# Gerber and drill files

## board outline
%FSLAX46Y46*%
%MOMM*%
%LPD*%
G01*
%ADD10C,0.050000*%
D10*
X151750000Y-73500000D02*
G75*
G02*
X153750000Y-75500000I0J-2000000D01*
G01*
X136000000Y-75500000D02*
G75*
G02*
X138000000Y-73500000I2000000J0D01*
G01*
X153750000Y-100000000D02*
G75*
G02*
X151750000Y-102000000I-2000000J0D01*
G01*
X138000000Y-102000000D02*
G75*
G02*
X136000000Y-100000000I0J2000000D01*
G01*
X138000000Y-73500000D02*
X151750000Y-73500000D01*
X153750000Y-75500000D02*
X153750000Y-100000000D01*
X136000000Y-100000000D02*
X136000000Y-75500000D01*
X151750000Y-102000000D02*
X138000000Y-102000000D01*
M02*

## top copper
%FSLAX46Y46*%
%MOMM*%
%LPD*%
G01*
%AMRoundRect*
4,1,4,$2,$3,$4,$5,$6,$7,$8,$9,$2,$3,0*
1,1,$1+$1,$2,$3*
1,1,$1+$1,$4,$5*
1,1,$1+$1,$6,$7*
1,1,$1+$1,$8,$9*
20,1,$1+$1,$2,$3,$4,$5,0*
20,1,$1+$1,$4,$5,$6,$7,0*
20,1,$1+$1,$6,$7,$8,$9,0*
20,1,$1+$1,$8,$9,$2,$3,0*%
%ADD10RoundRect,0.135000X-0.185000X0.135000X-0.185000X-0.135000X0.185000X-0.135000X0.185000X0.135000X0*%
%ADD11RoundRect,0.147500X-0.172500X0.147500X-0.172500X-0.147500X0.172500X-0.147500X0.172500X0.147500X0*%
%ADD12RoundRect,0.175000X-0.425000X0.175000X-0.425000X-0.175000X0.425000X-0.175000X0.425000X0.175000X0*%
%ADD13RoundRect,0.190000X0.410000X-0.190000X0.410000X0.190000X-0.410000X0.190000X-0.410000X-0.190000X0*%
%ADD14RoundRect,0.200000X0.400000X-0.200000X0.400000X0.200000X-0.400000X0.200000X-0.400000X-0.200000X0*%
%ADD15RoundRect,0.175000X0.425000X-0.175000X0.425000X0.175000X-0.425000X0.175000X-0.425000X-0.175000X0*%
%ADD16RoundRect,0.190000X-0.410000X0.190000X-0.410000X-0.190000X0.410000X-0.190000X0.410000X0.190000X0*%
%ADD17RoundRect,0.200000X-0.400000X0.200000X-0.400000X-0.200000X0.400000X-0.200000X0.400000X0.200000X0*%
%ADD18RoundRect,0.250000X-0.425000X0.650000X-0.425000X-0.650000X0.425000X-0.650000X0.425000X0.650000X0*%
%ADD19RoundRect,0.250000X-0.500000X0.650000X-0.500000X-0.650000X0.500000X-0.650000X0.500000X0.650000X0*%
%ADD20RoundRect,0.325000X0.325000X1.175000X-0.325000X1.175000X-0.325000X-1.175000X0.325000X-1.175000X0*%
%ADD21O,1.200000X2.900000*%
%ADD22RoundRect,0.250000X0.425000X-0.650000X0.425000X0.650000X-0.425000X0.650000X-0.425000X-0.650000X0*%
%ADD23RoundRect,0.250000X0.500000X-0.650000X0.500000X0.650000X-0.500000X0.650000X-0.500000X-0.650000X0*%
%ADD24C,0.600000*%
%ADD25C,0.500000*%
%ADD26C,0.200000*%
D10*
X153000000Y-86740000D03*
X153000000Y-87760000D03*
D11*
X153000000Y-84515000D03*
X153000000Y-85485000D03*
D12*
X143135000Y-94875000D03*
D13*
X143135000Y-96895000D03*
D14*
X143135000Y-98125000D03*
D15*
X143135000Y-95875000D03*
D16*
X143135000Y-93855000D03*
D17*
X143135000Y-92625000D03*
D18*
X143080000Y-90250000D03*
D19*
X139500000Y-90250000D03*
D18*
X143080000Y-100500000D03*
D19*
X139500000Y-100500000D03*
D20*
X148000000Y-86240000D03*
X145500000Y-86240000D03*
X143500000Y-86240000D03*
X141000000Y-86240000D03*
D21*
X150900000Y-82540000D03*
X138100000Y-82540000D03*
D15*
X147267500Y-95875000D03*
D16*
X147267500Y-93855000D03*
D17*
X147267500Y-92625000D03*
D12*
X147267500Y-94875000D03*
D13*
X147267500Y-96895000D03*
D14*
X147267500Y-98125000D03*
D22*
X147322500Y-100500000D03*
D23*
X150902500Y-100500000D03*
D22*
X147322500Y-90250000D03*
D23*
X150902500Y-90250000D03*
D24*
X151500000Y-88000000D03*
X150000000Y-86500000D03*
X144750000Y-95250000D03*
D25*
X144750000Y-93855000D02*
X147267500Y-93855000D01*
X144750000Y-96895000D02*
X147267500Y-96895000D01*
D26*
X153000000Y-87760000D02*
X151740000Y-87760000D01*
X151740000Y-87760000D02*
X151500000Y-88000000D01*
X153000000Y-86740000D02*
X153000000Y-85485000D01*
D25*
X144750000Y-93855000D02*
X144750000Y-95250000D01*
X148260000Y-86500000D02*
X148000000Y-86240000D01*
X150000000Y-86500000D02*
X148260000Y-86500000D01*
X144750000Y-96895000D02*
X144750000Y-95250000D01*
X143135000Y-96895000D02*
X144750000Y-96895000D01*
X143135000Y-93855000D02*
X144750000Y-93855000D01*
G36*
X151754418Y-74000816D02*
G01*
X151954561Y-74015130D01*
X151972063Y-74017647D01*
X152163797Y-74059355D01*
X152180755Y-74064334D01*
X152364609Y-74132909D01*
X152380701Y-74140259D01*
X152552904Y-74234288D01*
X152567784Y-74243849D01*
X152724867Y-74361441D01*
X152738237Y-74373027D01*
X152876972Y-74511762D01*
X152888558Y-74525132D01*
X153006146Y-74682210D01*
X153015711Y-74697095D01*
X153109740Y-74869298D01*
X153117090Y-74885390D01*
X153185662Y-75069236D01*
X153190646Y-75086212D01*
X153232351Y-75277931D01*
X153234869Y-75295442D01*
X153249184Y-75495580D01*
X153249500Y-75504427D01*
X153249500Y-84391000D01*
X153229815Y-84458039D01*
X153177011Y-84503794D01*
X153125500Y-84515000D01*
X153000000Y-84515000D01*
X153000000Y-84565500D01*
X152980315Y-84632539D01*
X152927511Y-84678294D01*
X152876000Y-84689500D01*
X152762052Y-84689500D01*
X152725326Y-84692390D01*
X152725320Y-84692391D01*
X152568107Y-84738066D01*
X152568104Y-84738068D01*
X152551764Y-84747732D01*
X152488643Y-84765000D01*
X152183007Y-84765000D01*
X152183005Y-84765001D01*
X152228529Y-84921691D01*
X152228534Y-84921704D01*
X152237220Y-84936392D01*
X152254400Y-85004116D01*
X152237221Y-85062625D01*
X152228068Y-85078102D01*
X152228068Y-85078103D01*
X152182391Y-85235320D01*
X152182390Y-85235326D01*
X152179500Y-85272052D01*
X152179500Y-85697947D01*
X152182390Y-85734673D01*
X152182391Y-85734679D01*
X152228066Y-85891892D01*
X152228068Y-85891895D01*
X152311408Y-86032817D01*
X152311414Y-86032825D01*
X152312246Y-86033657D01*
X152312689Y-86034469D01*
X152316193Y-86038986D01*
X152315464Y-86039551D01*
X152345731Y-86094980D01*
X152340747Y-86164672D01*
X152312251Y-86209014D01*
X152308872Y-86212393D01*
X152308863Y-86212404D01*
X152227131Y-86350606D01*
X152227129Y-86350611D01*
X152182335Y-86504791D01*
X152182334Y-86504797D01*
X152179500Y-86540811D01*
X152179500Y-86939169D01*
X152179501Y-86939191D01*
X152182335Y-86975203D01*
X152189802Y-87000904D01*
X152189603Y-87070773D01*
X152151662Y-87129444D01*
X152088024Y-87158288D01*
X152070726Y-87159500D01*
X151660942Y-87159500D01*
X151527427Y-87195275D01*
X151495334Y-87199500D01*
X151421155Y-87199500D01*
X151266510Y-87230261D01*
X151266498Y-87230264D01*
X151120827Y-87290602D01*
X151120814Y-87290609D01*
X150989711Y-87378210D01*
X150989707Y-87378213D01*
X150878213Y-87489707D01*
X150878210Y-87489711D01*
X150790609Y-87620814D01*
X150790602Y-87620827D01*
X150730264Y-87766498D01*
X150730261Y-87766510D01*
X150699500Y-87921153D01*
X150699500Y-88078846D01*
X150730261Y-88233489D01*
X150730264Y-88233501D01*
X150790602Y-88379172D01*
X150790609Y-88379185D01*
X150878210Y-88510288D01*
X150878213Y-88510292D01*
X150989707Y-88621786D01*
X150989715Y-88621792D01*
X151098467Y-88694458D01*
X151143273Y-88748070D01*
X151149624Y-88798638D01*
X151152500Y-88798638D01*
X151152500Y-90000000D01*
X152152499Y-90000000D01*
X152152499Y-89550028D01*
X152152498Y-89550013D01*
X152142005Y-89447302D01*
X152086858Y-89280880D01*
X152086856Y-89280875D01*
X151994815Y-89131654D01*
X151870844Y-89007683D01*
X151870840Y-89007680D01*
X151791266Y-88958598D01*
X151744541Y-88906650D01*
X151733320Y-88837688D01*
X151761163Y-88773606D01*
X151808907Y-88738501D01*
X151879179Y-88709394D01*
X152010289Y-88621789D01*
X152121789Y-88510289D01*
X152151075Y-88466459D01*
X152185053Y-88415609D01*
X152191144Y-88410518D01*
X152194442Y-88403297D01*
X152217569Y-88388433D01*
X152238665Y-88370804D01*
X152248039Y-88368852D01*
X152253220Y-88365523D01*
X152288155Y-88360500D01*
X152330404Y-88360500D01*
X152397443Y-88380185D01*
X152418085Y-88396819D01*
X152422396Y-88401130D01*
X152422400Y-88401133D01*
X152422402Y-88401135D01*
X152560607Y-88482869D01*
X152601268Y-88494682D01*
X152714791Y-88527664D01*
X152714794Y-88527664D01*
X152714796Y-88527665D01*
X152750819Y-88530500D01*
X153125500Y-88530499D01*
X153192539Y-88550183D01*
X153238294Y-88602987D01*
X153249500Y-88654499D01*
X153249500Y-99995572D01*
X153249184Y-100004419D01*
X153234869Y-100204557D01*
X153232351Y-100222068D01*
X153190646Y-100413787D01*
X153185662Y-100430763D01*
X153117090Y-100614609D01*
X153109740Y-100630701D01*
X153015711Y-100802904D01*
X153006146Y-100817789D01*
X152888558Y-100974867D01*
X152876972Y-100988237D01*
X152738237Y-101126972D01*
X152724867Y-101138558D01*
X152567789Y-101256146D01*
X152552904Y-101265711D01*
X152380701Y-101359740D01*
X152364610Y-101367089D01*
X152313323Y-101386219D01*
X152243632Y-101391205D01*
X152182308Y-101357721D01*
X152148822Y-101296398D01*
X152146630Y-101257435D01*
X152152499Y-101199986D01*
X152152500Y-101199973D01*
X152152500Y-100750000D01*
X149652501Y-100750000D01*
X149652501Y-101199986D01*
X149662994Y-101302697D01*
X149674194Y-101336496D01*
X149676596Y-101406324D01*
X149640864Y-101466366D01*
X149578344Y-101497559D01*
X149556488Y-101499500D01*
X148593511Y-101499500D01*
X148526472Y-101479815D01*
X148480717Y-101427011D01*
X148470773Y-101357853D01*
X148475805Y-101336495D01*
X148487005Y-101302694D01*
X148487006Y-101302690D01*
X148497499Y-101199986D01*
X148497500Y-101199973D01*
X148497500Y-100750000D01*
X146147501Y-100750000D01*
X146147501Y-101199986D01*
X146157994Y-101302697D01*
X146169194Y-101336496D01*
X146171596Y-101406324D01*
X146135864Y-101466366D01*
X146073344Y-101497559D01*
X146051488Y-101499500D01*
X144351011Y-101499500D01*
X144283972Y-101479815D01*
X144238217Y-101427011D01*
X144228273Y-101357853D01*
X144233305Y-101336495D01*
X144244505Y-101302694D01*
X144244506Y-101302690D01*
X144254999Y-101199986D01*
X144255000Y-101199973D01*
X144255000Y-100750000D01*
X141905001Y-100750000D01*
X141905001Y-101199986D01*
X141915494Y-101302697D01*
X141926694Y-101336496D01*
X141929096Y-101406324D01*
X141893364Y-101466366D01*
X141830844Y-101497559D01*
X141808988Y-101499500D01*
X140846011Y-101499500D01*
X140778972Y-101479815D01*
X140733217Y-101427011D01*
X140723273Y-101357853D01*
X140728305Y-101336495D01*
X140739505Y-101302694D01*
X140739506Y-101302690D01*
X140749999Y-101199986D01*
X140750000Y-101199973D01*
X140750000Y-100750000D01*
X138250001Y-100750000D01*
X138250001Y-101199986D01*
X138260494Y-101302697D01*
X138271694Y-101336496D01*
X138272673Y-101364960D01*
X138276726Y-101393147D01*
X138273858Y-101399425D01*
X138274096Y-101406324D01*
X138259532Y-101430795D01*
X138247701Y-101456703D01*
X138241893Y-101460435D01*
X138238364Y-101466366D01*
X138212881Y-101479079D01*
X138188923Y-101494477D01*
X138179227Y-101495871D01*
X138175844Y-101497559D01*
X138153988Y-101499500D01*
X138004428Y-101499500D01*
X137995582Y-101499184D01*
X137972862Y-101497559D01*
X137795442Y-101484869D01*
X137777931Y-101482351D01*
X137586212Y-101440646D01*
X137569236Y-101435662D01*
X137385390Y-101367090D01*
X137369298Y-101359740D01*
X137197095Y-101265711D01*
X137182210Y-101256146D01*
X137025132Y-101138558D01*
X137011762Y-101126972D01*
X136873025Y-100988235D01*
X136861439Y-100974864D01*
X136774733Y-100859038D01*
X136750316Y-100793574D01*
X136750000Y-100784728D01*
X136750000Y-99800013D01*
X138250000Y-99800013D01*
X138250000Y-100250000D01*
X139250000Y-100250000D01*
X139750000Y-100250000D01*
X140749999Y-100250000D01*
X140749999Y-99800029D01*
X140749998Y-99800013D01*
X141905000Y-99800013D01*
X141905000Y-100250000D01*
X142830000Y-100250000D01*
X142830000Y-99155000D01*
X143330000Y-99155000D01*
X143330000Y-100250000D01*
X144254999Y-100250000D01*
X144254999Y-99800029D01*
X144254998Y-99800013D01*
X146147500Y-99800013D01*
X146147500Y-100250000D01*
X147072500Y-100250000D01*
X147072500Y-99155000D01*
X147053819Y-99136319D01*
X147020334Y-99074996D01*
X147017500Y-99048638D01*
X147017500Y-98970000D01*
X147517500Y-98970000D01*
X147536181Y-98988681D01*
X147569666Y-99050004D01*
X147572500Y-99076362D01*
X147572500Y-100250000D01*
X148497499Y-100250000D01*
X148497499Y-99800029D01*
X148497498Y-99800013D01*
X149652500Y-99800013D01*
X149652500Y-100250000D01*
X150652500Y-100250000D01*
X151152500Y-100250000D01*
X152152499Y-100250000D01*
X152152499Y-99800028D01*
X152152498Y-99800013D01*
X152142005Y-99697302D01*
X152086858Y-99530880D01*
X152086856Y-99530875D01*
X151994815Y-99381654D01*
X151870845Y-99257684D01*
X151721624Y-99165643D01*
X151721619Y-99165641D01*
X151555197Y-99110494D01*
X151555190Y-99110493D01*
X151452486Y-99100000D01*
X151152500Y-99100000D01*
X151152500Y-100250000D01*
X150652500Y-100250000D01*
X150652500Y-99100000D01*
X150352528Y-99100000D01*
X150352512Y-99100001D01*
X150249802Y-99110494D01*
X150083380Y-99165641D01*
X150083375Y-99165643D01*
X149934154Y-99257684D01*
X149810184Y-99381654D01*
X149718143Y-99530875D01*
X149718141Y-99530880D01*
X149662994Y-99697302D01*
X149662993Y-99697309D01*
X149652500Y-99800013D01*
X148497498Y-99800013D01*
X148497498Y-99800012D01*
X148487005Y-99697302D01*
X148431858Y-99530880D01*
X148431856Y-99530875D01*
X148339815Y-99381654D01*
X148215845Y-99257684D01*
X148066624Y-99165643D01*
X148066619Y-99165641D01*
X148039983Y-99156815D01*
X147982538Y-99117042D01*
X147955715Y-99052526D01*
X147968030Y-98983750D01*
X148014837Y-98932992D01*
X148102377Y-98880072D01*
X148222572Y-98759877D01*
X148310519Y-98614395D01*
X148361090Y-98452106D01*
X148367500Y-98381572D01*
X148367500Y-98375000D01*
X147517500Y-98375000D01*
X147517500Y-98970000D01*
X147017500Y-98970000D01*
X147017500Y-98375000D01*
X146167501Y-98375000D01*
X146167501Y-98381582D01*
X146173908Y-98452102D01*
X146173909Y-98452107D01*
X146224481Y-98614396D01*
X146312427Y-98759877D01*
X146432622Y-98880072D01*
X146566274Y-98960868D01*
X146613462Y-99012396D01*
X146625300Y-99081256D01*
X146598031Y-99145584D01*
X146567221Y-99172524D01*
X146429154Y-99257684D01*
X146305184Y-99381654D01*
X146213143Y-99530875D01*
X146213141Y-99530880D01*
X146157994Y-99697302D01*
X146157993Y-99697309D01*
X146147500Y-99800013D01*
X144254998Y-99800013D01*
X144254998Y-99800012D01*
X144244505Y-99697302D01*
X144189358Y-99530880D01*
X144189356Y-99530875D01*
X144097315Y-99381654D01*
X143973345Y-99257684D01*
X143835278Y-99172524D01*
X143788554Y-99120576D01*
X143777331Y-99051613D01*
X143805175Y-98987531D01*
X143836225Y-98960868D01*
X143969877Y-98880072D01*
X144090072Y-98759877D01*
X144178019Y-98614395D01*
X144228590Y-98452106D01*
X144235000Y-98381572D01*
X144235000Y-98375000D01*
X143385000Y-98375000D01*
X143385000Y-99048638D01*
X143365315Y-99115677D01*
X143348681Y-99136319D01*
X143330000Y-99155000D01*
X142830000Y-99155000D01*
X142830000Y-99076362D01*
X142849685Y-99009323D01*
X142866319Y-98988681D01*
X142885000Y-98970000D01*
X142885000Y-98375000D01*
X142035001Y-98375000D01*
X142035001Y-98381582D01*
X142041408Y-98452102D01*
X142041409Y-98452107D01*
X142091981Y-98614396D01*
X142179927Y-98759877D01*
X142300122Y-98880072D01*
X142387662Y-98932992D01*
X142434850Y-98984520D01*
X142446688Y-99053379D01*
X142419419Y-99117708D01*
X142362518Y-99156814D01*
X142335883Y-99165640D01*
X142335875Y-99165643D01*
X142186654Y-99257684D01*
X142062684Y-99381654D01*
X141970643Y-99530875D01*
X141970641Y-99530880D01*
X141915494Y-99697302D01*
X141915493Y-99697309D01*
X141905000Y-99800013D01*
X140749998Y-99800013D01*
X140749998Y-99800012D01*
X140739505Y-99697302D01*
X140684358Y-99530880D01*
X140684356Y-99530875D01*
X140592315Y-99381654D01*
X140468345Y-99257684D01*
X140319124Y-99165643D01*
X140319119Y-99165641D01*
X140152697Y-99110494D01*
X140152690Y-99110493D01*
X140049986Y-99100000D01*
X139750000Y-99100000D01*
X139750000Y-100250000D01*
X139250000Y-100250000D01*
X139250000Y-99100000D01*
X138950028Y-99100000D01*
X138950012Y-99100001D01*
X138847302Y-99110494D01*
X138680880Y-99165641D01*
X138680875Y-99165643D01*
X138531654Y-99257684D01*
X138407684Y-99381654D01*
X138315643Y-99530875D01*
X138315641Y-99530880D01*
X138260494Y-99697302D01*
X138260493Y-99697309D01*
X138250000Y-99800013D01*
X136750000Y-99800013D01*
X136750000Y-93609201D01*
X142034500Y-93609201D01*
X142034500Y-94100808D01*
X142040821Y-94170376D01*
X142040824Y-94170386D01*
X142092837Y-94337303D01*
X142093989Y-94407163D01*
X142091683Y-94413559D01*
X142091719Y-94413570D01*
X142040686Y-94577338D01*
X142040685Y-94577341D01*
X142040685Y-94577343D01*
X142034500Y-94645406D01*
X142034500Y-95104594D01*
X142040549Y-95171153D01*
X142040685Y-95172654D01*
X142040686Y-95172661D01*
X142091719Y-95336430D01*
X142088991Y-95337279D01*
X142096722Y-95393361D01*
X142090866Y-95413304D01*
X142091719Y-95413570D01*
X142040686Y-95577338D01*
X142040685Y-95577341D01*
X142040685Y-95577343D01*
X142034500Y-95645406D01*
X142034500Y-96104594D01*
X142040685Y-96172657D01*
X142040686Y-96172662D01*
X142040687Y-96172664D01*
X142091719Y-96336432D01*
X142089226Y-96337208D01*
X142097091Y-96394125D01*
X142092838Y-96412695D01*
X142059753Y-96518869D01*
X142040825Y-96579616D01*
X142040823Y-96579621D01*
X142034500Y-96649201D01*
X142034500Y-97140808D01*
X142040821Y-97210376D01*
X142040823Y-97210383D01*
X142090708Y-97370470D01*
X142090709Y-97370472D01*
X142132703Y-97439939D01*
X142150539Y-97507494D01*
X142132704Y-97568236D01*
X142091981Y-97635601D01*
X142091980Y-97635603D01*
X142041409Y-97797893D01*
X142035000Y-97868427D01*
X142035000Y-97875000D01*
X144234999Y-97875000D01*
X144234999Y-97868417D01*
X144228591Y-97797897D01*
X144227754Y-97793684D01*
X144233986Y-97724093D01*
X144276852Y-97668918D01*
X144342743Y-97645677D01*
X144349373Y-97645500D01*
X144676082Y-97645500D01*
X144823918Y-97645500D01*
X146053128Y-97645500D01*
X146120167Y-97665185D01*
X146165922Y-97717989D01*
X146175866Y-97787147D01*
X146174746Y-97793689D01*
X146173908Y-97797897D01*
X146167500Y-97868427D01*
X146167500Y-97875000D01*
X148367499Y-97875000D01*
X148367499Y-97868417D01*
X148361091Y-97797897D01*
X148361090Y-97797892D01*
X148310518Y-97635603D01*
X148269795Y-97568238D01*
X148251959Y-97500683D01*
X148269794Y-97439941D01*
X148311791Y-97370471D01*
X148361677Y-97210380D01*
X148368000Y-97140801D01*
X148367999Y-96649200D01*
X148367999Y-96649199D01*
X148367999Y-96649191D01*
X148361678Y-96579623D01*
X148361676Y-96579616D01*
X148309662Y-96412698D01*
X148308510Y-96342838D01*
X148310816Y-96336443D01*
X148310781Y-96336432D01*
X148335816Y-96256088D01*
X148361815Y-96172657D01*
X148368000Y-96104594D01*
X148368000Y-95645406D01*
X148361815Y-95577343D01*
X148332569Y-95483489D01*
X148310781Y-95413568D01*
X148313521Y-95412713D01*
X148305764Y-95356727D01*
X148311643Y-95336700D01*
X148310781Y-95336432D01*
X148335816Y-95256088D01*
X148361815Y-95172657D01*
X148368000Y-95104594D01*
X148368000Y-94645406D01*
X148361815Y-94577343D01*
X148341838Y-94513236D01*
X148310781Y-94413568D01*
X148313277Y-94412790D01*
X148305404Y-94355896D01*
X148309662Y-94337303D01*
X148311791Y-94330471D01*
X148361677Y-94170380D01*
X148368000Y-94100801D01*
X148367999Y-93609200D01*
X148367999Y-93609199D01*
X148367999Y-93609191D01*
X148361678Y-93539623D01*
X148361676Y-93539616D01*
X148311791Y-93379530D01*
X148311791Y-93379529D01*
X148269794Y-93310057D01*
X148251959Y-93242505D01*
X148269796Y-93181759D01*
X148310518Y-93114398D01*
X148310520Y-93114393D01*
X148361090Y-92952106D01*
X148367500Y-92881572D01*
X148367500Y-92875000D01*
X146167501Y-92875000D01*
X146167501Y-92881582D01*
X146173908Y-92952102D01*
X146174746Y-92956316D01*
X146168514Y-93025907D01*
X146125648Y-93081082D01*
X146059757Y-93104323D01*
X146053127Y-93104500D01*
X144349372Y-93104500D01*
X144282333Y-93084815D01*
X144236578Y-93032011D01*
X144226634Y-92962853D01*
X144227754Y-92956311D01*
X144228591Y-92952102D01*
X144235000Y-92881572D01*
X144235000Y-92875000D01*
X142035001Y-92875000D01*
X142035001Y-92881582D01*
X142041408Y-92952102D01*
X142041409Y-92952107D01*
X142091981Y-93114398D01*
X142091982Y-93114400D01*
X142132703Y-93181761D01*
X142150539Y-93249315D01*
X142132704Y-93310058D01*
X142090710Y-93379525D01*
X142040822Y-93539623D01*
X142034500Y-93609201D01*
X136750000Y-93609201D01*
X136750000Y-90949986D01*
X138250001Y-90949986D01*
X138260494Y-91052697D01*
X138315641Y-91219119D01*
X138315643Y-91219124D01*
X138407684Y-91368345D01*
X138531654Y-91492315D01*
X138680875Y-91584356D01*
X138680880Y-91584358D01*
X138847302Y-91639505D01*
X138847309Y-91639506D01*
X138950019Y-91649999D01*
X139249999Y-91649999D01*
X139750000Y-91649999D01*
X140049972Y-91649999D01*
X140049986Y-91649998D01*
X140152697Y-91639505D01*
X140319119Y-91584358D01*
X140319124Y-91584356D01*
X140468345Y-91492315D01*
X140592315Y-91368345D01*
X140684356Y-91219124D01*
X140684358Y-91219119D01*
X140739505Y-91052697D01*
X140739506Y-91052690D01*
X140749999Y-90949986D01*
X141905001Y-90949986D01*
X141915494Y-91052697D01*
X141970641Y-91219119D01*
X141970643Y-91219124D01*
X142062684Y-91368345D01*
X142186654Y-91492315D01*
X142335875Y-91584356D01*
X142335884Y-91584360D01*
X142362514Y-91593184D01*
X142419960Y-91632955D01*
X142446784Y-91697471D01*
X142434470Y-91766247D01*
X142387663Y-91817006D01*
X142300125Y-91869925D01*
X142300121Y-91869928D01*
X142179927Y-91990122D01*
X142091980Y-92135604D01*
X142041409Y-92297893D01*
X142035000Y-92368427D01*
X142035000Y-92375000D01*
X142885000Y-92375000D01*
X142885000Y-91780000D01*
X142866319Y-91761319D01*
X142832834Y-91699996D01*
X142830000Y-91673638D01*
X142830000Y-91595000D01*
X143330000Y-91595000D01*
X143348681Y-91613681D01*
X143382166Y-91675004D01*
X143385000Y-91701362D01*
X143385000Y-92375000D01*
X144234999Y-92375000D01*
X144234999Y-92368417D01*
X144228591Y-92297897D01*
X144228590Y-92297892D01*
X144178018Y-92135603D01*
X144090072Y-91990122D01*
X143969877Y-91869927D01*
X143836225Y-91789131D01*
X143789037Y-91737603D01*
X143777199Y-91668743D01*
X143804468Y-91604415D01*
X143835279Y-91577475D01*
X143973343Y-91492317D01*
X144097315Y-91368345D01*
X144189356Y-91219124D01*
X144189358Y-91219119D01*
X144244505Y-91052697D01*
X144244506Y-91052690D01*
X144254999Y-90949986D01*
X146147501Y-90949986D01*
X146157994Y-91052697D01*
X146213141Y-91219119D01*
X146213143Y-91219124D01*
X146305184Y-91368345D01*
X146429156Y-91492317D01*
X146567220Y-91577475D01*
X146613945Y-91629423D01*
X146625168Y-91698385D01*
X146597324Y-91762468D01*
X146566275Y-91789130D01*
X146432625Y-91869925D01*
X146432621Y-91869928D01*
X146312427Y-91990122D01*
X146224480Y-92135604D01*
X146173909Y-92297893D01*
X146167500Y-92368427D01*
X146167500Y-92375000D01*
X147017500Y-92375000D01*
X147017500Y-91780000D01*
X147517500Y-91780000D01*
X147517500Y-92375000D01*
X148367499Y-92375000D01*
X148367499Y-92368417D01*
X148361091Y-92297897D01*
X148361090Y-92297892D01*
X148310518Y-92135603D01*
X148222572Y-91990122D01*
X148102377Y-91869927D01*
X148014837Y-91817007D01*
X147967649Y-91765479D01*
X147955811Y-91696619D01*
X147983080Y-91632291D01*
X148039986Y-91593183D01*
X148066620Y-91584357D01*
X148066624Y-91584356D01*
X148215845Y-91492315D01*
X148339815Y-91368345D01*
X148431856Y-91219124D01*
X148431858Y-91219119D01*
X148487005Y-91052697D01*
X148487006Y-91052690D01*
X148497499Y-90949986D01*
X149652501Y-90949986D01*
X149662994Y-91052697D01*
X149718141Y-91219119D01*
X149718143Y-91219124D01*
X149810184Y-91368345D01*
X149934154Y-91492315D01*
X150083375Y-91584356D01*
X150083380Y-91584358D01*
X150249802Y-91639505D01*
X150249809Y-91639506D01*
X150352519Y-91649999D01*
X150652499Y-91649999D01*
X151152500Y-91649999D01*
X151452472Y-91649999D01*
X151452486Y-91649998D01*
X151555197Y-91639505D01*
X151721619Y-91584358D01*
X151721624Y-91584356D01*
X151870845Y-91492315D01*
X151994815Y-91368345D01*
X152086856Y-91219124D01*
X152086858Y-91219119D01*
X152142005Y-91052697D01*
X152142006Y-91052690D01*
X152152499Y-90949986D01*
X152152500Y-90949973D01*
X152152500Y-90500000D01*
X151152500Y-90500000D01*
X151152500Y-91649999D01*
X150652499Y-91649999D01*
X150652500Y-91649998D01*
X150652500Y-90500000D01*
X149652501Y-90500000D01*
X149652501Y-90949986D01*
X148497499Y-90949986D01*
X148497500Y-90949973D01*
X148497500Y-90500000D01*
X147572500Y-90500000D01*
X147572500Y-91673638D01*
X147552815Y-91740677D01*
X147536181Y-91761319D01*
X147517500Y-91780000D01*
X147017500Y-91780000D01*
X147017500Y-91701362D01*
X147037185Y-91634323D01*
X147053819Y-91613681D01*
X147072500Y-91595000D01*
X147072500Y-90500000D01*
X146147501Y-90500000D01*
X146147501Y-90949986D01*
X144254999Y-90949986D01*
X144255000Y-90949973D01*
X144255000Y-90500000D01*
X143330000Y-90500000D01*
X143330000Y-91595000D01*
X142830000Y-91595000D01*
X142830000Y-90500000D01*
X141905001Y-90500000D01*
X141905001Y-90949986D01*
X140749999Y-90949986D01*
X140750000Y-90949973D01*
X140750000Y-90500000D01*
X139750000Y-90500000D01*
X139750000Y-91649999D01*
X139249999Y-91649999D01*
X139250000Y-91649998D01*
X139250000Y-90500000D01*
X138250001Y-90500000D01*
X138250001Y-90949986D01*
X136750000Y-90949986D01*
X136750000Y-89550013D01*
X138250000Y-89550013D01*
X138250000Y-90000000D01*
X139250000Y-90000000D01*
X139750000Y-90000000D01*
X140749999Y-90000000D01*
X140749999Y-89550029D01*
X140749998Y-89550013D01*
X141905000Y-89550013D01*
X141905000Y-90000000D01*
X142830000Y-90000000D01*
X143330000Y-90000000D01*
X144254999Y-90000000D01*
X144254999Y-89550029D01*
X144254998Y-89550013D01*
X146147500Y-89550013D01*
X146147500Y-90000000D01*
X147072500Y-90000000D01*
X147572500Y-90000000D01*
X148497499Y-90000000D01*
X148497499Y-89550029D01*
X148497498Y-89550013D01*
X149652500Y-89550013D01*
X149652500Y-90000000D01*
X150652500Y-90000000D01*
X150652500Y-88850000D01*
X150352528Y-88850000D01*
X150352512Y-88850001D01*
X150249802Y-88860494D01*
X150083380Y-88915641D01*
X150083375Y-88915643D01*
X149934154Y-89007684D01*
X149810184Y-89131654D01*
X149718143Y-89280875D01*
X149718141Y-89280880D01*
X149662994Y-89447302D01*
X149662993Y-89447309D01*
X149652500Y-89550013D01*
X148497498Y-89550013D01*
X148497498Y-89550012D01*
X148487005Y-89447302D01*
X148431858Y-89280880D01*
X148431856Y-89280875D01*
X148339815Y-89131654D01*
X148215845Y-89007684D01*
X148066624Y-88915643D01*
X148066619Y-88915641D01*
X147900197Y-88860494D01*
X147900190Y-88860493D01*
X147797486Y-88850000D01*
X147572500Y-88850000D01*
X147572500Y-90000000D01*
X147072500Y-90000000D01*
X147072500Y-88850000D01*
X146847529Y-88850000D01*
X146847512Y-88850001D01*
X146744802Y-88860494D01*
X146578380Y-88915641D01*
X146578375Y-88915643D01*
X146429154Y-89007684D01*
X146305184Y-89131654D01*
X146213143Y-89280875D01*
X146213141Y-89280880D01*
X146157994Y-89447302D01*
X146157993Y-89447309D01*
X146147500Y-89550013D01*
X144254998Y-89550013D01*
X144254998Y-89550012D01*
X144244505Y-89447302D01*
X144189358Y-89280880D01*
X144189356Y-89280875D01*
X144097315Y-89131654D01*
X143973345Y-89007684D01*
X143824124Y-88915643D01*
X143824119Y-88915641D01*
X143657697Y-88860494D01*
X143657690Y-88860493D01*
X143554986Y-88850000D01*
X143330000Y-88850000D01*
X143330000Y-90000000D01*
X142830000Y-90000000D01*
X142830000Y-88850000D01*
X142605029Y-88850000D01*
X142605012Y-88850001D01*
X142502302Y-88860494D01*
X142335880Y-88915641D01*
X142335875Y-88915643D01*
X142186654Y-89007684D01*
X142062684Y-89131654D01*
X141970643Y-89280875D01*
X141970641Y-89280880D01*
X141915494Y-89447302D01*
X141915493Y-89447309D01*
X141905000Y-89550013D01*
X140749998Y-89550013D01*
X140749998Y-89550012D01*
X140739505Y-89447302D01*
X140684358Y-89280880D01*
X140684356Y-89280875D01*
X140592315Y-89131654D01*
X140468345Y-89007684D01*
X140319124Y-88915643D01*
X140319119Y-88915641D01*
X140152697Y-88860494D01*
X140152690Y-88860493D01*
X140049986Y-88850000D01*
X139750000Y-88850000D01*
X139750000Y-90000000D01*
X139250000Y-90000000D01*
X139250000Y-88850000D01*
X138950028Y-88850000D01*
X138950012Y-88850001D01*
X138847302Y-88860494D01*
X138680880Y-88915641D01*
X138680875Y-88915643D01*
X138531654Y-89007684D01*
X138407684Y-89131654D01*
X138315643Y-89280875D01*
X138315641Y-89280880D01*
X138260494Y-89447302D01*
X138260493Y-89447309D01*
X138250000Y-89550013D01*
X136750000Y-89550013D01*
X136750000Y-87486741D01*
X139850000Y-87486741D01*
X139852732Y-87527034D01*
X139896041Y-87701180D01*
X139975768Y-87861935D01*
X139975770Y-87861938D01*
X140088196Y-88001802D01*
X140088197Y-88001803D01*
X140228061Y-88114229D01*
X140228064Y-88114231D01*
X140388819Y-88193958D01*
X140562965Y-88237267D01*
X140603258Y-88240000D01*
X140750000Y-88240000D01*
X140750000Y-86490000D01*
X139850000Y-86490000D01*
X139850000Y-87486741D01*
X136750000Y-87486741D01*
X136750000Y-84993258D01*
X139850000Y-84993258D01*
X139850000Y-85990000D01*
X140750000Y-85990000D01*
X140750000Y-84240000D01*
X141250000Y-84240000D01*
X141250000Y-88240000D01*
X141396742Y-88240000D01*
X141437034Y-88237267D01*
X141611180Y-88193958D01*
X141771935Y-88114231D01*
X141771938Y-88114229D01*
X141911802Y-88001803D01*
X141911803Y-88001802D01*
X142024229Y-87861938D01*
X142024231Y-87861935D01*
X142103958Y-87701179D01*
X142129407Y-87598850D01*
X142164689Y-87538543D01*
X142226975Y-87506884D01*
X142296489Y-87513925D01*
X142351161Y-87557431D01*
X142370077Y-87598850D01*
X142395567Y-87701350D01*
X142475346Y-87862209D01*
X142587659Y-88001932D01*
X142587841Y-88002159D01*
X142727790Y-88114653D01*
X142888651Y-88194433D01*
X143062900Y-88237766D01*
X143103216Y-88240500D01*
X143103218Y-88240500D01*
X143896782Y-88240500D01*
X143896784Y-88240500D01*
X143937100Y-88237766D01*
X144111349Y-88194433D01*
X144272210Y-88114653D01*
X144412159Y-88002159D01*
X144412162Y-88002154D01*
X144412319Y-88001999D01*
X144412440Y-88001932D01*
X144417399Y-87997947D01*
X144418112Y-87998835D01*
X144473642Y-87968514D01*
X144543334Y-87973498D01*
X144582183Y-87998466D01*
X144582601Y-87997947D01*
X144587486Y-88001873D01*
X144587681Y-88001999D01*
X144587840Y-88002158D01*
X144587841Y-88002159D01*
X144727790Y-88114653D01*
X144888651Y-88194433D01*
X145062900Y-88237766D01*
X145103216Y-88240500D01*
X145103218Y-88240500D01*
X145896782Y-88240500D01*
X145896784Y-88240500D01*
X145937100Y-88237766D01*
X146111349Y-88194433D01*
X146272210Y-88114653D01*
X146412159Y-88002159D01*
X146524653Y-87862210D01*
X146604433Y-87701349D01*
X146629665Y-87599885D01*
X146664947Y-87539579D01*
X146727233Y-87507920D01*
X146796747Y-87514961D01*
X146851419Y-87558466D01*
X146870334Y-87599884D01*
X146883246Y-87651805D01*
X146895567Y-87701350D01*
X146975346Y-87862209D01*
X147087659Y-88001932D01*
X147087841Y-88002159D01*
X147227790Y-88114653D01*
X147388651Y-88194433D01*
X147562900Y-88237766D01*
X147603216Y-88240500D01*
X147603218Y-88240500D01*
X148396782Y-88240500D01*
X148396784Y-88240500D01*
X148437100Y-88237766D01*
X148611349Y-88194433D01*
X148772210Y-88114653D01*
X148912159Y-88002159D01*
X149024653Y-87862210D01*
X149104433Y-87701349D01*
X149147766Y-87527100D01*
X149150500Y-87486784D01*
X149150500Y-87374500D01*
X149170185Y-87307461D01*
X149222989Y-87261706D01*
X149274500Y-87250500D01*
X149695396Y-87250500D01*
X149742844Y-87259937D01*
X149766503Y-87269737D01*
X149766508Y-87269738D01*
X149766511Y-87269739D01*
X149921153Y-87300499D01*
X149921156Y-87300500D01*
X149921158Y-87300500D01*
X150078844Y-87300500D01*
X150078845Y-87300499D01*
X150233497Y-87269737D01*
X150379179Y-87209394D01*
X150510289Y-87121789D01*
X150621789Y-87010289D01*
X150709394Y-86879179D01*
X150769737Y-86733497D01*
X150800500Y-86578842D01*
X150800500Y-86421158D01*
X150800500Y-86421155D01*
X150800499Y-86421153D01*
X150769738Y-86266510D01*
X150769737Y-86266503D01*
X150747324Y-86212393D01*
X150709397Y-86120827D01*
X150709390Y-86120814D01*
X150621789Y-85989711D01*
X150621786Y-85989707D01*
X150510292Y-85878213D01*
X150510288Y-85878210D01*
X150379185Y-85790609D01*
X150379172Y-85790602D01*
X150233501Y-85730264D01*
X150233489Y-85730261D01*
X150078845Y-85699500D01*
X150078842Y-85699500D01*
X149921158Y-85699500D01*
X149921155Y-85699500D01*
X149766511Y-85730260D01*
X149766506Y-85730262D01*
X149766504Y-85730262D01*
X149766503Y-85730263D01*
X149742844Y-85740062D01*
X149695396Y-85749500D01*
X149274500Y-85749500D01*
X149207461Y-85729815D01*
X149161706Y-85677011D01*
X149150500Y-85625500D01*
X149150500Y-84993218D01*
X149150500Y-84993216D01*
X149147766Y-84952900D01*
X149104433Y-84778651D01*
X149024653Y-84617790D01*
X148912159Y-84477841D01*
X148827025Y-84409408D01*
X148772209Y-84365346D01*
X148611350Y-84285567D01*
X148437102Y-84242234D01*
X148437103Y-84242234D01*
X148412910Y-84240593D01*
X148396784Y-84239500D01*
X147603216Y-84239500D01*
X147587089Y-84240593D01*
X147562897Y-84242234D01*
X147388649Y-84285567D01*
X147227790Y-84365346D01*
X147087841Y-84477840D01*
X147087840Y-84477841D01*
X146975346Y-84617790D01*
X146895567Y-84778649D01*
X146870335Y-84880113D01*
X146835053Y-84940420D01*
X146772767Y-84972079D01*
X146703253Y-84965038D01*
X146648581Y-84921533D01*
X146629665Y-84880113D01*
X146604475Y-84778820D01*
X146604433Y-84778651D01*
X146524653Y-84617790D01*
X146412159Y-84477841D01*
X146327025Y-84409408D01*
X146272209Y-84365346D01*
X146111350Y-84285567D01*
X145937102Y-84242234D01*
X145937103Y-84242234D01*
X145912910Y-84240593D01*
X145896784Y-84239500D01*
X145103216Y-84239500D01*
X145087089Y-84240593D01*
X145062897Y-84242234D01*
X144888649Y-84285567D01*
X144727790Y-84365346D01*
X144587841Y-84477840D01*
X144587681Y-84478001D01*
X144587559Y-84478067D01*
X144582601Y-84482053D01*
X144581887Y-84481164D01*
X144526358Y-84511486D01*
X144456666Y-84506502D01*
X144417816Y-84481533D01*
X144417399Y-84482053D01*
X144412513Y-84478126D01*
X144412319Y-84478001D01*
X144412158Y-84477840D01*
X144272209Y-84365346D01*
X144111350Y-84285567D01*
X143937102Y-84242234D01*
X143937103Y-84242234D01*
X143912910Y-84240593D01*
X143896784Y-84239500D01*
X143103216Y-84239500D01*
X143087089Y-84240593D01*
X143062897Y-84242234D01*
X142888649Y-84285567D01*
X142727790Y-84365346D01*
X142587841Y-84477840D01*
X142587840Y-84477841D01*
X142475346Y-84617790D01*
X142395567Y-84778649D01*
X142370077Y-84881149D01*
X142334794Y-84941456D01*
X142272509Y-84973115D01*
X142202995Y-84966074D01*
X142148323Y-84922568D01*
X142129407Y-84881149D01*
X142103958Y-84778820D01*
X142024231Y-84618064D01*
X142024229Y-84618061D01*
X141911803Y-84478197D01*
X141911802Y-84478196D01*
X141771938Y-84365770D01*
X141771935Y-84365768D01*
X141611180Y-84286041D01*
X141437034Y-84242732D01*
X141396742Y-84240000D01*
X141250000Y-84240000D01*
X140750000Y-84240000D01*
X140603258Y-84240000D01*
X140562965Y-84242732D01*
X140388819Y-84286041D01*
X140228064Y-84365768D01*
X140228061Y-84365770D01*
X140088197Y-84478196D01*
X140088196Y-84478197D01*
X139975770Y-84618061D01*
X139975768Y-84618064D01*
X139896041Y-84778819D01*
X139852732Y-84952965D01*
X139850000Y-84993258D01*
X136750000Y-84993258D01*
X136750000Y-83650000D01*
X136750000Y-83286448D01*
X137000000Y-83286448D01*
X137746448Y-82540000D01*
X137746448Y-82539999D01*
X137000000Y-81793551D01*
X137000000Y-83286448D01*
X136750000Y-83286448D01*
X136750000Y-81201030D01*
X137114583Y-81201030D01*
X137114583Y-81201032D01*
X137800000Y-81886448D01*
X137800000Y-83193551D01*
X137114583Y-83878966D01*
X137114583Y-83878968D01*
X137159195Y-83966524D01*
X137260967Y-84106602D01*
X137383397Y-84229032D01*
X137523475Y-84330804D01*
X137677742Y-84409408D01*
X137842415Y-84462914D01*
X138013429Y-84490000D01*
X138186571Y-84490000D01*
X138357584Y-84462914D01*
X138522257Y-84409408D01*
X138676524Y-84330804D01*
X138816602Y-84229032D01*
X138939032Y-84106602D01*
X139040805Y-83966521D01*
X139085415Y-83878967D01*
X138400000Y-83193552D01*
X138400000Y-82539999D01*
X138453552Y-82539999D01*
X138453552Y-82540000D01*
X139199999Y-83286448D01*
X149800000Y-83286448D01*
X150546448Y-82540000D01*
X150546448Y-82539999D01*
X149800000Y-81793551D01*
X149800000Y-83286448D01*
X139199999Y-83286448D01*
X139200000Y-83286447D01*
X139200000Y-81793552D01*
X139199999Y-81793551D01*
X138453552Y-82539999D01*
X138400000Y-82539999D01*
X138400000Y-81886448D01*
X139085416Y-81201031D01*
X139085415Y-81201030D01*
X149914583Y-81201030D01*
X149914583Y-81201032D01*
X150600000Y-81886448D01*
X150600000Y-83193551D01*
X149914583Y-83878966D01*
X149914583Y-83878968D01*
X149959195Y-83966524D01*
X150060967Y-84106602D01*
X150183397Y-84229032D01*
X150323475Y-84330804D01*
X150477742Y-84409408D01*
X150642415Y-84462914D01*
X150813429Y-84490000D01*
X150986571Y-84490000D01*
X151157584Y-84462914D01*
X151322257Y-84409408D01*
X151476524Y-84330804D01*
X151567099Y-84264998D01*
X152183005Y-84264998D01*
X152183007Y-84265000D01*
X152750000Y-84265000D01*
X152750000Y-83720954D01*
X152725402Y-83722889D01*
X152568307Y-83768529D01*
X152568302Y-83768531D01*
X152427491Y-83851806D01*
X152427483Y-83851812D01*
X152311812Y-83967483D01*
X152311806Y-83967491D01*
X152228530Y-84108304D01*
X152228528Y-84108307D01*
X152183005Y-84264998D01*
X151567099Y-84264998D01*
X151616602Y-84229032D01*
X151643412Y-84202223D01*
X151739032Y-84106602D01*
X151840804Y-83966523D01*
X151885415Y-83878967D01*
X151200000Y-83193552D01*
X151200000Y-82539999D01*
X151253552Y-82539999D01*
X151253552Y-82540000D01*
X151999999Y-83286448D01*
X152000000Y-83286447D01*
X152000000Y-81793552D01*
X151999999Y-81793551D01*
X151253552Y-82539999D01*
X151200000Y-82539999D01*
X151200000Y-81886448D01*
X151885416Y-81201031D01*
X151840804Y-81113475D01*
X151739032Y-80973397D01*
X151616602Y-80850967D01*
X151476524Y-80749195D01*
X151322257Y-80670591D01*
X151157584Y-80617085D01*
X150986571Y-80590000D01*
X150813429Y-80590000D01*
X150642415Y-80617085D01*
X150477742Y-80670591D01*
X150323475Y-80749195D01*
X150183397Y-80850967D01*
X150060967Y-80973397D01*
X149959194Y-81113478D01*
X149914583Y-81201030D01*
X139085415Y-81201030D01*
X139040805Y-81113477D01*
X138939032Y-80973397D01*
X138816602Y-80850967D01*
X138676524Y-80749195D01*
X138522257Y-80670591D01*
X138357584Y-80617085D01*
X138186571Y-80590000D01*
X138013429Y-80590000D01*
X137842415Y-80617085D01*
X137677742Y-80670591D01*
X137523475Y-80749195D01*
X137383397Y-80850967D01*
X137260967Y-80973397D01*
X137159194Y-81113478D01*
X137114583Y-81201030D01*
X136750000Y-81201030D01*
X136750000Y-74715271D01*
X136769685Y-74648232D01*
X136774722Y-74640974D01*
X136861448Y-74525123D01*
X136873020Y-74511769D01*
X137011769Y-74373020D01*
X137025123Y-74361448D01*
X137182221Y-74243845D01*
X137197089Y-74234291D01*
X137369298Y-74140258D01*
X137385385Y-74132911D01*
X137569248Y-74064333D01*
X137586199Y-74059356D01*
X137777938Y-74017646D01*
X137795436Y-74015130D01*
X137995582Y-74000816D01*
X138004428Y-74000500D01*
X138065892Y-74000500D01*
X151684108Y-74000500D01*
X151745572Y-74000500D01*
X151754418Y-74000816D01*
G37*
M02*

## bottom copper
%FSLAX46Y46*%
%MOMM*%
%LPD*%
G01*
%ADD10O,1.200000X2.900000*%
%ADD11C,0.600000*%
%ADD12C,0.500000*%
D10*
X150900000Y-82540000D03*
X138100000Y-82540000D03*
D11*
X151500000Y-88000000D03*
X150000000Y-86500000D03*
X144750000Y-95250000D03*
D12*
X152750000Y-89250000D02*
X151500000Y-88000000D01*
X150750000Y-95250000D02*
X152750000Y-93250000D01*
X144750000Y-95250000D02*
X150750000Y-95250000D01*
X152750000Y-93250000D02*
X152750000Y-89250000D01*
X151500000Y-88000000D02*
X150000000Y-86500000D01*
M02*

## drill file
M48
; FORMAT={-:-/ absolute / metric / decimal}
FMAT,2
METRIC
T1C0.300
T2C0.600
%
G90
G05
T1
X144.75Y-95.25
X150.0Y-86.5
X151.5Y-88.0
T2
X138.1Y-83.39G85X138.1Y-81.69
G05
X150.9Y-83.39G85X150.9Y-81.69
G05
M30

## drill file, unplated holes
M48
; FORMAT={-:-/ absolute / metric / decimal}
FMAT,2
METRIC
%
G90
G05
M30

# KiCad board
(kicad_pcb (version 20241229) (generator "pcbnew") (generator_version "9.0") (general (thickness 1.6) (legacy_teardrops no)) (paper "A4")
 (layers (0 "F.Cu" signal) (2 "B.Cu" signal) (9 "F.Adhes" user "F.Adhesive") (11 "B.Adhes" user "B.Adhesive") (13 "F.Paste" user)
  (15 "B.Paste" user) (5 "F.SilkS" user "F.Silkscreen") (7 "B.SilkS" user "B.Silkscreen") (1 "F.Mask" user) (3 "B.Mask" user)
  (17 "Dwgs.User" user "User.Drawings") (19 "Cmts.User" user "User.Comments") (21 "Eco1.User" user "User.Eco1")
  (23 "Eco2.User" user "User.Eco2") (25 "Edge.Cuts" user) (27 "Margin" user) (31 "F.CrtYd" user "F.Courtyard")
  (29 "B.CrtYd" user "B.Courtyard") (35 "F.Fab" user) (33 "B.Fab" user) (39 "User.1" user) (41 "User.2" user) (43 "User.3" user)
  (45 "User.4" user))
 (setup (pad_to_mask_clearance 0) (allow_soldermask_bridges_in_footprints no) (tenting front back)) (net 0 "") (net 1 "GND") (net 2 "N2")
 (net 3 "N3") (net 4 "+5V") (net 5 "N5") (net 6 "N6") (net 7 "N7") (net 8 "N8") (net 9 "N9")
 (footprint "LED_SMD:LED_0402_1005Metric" (layer "F.Cu") (at 153 85 -90)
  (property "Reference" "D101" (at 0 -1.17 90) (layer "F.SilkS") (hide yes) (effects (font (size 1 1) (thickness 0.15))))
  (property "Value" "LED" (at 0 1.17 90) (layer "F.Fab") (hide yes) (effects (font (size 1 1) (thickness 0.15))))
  (pad "1" smd roundrect (at -0.485 0 270) (size 0.59 0.64) (layers "F.Cu" "F.Mask" "F.Paste") (roundrect_rratio 0.25) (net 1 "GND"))
  (pad "2" smd roundrect (at 0.485 0 270) (size 0.59 0.64) (layers "F.Cu" "F.Mask" "F.Paste") (roundrect_rratio 0.25) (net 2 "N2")))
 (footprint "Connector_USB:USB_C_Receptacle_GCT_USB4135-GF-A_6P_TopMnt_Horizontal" (layer "F.Cu") (at 150.3 95.375 90)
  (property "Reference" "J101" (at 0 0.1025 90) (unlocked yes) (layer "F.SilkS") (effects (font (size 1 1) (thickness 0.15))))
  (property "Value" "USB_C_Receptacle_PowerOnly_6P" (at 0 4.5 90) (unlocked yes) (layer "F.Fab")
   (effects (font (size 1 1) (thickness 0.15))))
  (pad "A5" smd roundrect (at -0.5 -3.0325 90) (size 0.7 1.2) (layers "F.Cu" "F.Mask" "F.Paste") (roundrect_rratio 0.25) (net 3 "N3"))
  (pad "A9" smd roundrect (at 1.52 -3.0325 270) (size 0.76 1.2) (layers "F.Cu" "F.Mask" "F.Paste") (roundrect_rratio 0.25) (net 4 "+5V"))
  (pad "A12" smd roundrect (at 2.75 -3.0325 270) (size 0.8 1.2) (layers "F.Cu" "F.Mask" "F.Paste") (roundrect_rratio 0.25) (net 1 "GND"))
  (pad "B5" smd roundrect (at 0.5 -3.0325 270) (size 0.7 1.2) (layers "F.Cu" "F.Mask" "F.Paste") (roundrect_rratio 0.25) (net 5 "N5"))
  (pad "B9" smd roundrect (at -1.52 -3.0325 90) (size 0.76 1.2) (layers "F.Cu" "F.Mask" "F.Paste") (roundrect_rratio 0.25) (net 4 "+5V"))
  (pad "B12" smd roundrect (at -2.75 -3.0325 90) (size 0.8 1.2) (layers "F.Cu" "F.Mask" "F.Paste") (roundrect_rratio 0.25) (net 1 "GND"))
  (pad "S1" smd roundrect (at -5.125 -2.9775 90) (size 1.8 1.35) (layers "F.Cu" "F.Mask" "F.Paste") (roundrect_rratio 0.1851851852)
   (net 1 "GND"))
  (pad "S1" smd roundrect (at -5.125 0.6025 90) (size 1.8 1.5) (layers "F.Cu" "F.Mask" "F.Paste") (roundrect_rratio 0.1666666667)
   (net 1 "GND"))
  (pad "S1" smd roundrect (at 5.125 -2.9775 90) (size 1.8 1.35) (layers "F.Cu" "F.Mask" "F.Paste") (roundrect_rratio 0.1851851852)
   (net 1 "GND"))
  (pad "S1" smd roundrect (at 5.125 0.6025 90) (size 1.8 1.5) (layers "F.Cu" "F.Mask" "F.Paste") (roundrect_rratio 0.1666666667)
   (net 1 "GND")))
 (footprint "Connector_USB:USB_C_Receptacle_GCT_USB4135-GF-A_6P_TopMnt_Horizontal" (layer "F.Cu") (at 140.1025 95.375 -90)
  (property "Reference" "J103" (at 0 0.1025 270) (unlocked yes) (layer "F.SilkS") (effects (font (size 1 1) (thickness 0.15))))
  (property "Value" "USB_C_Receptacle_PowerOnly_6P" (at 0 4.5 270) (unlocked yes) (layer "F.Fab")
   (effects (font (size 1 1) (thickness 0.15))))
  (pad "A5" smd roundrect (at -0.5 -3.0325 270) (size 0.7 1.2) (layers "F.Cu" "F.Mask" "F.Paste") (roundrect_rratio 0.25) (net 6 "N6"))
  (pad "A9" smd roundrect (at 1.52 -3.0325 90) (size 0.76 1.2) (layers "F.Cu" "F.Mask" "F.Paste") (roundrect_rratio 0.25) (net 4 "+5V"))
  (pad "A12" smd roundrect (at 2.75 -3.0325 90) (size 0.8 1.2) (layers "F.Cu" "F.Mask" "F.Paste") (roundrect_rratio 0.25) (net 1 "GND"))
  (pad "B5" smd roundrect (at 0.5 -3.0325 90) (size 0.7 1.2) (layers "F.Cu" "F.Mask" "F.Paste") (roundrect_rratio 0.25) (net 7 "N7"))
  (pad "B9" smd roundrect (at -1.52 -3.0325 270) (size 0.76 1.2) (layers "F.Cu" "F.Mask" "F.Paste") (roundrect_rratio 0.25) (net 4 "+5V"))
  (pad "B12" smd roundrect (at -2.75 -3.0325 270) (size 0.8 1.2) (layers "F.Cu" "F.Mask" "F.Paste") (roundrect_rratio 0.25) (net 1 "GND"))
  (pad "S1" smd roundrect (at -5.125 -2.9775 270) (size 1.8 1.35) (layers "F.Cu" "F.Mask" "F.Paste") (roundrect_rratio 0.1851851852)
   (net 1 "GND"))
  (pad "S1" smd roundrect (at -5.125 0.6025 270) (size 1.8 1.5) (layers "F.Cu" "F.Mask" "F.Paste") (roundrect_rratio 0.1666666667)
   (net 1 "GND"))
  (pad "S1" smd roundrect (at 5.125 -2.9775 270) (size 1.8 1.35) (layers "F.Cu" "F.Mask" "F.Paste") (roundrect_rratio 0.1851851852)
   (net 1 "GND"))
  (pad "S1" smd roundrect (at 5.125 0.6025 270) (size 1.8 1.5) (layers "F.Cu" "F.Mask" "F.Paste") (roundrect_rratio 0.1666666667)
   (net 1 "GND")))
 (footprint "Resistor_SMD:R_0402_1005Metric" (layer "F.Cu") (at 153 87.25 -90)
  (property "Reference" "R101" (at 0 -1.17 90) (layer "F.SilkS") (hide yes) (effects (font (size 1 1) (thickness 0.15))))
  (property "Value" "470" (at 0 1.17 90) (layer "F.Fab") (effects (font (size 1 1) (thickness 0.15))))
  (pad "1" smd roundrect (at -0.51 0 270) (size 0.54 0.64) (layers "F.Cu" "F.Mask" "F.Paste") (roundrect_rratio 0.25) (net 2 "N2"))
  (pad "2" smd roundrect (at 0.51 0 270) (size 0.54 0.64) (layers "F.Cu" "F.Mask" "F.Paste") (roundrect_rratio 0.25) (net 4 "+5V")))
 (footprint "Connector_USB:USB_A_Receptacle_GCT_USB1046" (layer "F.Cu") (at 144.5 78.99 180)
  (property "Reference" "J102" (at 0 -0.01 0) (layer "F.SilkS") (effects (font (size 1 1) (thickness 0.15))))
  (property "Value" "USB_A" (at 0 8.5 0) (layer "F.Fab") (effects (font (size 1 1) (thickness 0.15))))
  (pad "" smd oval (at -6.4 -3.55 180) (size 1.2 2.9) (layers "F.Paste") (thermal_bridge_angle 45))
  (pad "" smd oval (at 6.4 -3.55 180) (size 1.2 2.9) (layers "F.Paste") (thermal_bridge_angle 45))
  (pad "1" smd roundrect (at -3.5 -7.25 180) (size 1.3 3) (layers "F.Cu" "F.Mask" "F.Paste") (roundrect_rratio 0.25) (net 4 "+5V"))
  (pad "2" smd roundrect (at -1 -7.25 180) (size 1.3 3) (layers "F.Cu" "F.Mask" "F.Paste") (roundrect_rratio 0.25) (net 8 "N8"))
  (pad "3" smd roundrect (at 1 -7.25 180) (size 1.3 3) (layers "F.Cu" "F.Mask" "F.Paste") (roundrect_rratio 0.25) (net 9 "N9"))
  (pad "4" smd roundrect (at 3.5 -7.25 180) (size 1.3 3) (layers "F.Cu" "F.Mask" "F.Paste") (roundrect_rratio 0.25) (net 1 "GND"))
  (pad "5" thru_hole oval (at -6.4 -3.55 180) (size 1.2 2.9) (drill oval 0.6 2.3) (layers "*.Cu" "*.Mask") (remove_unused_layers no)
   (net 1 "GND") (thermal_bridge_angle 45))
  (pad "5" thru_hole oval (at 6.4 -3.55 180) (size 1.2 2.9) (drill oval 0.6 2.3) (layers "*.Cu" "*.Mask") (remove_unused_layers no)
   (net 1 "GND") (thermal_bridge_angle 45)))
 (gr_line (start 153.75 75.5) (end 153.75 100) (stroke (width 0.05) (type default)) (layer "Edge.Cuts"))
 (gr_arc (start 136 75.5) (mid 136.585786 74.085786) (end 138 73.5) (stroke (width 0.05) (type default)) (layer "Edge.Cuts"))
 (gr_arc (start 153.75 100) (mid 153.164214 101.414214) (end 151.75 102) (stroke (width 0.05) (type default)) (layer "Edge.Cuts"))
 (gr_line (start 138 73.5) (end 151.75 73.5) (stroke (width 0.05) (type default)) (layer "Edge.Cuts"))
 (gr_arc (start 138 102) (mid 136.585786 101.414214) (end 136 100) (stroke (width 0.05) (type default)) (layer "Edge.Cuts"))
 (gr_line (start 136 100) (end 136 75.5) (stroke (width 0.05) (type default)) (layer "Edge.Cuts"))
 (gr_arc (start 151.75 73.5) (mid 153.164214 74.085786) (end 153.75 75.5) (stroke (width 0.05) (type default)) (layer "Edge.Cuts"))
 (gr_line (start 151.75 102) (end 138 102) (stroke (width 0.05) (type default)) (layer "Edge.Cuts"))
 (segment (start 144.75 96.895) (end 144.75 95.25) (width 0.5) (layer "F.Cu") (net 4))
 (segment (start 143.135 96.895) (end 144.75 96.895) (width 0.5) (layer "F.Cu") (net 4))
 (segment (start 143.135 93.855) (end 144.75 93.855) (width 0.5) (layer "F.Cu") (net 4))
 (segment (start 144.75 93.855) (end 144.75 95.25) (width 0.5) (layer "F.Cu") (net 4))
 (segment (start 144.75 96.895) (end 147.2675 96.895) (width 0.5) (layer "F.Cu") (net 4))
 (segment (start 153 87.76) (end 151.74 87.76) (width 0.2) (layer "F.Cu") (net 4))
 (segment (start 150 86.5) (end 148.26 86.5) (width 0.5) (layer "F.Cu") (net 4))
 (segment (start 148.26 86.5) (end 148 86.24) (width 0.5) (layer "F.Cu") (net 4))
 (segment (start 151.74 87.76) (end 151.5 88) (width 0.2) (layer "F.Cu") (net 4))
 (segment (start 144.75 93.855) (end 147.2675 93.855) (width 0.5) (layer "F.Cu") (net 4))
 (via (at 150 86.5) (size 0.6) (drill 0.3) (layers "F.Cu" "B.Cu") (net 4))
 (via (at 144.75 95.25) (size 0.6) (drill 0.3) (layers "F.Cu" "B.Cu") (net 4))
 (via (at 151.5 88) (size 0.6) (drill 0.3) (layers "F.Cu" "B.Cu") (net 4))
 (segment (start 152.75 89.25) (end 151.5 88) (width 0.5) (layer "B.Cu") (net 4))
 (segment (start 150.75 95.25) (end 152.75 93.25) (width 0.5) (layer "B.Cu") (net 4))
 (segment (start 151.5 88) (end 150 86.5) (width 0.5) (layer "B.Cu") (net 4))
 (segment (start 144.75 95.25) (end 150.75 95.25) (width 0.5) (layer "B.Cu") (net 4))
 (segment (start 152.75 93.25) (end 152.75 89.25) (width 0.5) (layer "B.Cu") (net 4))
 (segment (start 153 86.74) (end 153 85.485) (width 0.2) (layer "F.Cu") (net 2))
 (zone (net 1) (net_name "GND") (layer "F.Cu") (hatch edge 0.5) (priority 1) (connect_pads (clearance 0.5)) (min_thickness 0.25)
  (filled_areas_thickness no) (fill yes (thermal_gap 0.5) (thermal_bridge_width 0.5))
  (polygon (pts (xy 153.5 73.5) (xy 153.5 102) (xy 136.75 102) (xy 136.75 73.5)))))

